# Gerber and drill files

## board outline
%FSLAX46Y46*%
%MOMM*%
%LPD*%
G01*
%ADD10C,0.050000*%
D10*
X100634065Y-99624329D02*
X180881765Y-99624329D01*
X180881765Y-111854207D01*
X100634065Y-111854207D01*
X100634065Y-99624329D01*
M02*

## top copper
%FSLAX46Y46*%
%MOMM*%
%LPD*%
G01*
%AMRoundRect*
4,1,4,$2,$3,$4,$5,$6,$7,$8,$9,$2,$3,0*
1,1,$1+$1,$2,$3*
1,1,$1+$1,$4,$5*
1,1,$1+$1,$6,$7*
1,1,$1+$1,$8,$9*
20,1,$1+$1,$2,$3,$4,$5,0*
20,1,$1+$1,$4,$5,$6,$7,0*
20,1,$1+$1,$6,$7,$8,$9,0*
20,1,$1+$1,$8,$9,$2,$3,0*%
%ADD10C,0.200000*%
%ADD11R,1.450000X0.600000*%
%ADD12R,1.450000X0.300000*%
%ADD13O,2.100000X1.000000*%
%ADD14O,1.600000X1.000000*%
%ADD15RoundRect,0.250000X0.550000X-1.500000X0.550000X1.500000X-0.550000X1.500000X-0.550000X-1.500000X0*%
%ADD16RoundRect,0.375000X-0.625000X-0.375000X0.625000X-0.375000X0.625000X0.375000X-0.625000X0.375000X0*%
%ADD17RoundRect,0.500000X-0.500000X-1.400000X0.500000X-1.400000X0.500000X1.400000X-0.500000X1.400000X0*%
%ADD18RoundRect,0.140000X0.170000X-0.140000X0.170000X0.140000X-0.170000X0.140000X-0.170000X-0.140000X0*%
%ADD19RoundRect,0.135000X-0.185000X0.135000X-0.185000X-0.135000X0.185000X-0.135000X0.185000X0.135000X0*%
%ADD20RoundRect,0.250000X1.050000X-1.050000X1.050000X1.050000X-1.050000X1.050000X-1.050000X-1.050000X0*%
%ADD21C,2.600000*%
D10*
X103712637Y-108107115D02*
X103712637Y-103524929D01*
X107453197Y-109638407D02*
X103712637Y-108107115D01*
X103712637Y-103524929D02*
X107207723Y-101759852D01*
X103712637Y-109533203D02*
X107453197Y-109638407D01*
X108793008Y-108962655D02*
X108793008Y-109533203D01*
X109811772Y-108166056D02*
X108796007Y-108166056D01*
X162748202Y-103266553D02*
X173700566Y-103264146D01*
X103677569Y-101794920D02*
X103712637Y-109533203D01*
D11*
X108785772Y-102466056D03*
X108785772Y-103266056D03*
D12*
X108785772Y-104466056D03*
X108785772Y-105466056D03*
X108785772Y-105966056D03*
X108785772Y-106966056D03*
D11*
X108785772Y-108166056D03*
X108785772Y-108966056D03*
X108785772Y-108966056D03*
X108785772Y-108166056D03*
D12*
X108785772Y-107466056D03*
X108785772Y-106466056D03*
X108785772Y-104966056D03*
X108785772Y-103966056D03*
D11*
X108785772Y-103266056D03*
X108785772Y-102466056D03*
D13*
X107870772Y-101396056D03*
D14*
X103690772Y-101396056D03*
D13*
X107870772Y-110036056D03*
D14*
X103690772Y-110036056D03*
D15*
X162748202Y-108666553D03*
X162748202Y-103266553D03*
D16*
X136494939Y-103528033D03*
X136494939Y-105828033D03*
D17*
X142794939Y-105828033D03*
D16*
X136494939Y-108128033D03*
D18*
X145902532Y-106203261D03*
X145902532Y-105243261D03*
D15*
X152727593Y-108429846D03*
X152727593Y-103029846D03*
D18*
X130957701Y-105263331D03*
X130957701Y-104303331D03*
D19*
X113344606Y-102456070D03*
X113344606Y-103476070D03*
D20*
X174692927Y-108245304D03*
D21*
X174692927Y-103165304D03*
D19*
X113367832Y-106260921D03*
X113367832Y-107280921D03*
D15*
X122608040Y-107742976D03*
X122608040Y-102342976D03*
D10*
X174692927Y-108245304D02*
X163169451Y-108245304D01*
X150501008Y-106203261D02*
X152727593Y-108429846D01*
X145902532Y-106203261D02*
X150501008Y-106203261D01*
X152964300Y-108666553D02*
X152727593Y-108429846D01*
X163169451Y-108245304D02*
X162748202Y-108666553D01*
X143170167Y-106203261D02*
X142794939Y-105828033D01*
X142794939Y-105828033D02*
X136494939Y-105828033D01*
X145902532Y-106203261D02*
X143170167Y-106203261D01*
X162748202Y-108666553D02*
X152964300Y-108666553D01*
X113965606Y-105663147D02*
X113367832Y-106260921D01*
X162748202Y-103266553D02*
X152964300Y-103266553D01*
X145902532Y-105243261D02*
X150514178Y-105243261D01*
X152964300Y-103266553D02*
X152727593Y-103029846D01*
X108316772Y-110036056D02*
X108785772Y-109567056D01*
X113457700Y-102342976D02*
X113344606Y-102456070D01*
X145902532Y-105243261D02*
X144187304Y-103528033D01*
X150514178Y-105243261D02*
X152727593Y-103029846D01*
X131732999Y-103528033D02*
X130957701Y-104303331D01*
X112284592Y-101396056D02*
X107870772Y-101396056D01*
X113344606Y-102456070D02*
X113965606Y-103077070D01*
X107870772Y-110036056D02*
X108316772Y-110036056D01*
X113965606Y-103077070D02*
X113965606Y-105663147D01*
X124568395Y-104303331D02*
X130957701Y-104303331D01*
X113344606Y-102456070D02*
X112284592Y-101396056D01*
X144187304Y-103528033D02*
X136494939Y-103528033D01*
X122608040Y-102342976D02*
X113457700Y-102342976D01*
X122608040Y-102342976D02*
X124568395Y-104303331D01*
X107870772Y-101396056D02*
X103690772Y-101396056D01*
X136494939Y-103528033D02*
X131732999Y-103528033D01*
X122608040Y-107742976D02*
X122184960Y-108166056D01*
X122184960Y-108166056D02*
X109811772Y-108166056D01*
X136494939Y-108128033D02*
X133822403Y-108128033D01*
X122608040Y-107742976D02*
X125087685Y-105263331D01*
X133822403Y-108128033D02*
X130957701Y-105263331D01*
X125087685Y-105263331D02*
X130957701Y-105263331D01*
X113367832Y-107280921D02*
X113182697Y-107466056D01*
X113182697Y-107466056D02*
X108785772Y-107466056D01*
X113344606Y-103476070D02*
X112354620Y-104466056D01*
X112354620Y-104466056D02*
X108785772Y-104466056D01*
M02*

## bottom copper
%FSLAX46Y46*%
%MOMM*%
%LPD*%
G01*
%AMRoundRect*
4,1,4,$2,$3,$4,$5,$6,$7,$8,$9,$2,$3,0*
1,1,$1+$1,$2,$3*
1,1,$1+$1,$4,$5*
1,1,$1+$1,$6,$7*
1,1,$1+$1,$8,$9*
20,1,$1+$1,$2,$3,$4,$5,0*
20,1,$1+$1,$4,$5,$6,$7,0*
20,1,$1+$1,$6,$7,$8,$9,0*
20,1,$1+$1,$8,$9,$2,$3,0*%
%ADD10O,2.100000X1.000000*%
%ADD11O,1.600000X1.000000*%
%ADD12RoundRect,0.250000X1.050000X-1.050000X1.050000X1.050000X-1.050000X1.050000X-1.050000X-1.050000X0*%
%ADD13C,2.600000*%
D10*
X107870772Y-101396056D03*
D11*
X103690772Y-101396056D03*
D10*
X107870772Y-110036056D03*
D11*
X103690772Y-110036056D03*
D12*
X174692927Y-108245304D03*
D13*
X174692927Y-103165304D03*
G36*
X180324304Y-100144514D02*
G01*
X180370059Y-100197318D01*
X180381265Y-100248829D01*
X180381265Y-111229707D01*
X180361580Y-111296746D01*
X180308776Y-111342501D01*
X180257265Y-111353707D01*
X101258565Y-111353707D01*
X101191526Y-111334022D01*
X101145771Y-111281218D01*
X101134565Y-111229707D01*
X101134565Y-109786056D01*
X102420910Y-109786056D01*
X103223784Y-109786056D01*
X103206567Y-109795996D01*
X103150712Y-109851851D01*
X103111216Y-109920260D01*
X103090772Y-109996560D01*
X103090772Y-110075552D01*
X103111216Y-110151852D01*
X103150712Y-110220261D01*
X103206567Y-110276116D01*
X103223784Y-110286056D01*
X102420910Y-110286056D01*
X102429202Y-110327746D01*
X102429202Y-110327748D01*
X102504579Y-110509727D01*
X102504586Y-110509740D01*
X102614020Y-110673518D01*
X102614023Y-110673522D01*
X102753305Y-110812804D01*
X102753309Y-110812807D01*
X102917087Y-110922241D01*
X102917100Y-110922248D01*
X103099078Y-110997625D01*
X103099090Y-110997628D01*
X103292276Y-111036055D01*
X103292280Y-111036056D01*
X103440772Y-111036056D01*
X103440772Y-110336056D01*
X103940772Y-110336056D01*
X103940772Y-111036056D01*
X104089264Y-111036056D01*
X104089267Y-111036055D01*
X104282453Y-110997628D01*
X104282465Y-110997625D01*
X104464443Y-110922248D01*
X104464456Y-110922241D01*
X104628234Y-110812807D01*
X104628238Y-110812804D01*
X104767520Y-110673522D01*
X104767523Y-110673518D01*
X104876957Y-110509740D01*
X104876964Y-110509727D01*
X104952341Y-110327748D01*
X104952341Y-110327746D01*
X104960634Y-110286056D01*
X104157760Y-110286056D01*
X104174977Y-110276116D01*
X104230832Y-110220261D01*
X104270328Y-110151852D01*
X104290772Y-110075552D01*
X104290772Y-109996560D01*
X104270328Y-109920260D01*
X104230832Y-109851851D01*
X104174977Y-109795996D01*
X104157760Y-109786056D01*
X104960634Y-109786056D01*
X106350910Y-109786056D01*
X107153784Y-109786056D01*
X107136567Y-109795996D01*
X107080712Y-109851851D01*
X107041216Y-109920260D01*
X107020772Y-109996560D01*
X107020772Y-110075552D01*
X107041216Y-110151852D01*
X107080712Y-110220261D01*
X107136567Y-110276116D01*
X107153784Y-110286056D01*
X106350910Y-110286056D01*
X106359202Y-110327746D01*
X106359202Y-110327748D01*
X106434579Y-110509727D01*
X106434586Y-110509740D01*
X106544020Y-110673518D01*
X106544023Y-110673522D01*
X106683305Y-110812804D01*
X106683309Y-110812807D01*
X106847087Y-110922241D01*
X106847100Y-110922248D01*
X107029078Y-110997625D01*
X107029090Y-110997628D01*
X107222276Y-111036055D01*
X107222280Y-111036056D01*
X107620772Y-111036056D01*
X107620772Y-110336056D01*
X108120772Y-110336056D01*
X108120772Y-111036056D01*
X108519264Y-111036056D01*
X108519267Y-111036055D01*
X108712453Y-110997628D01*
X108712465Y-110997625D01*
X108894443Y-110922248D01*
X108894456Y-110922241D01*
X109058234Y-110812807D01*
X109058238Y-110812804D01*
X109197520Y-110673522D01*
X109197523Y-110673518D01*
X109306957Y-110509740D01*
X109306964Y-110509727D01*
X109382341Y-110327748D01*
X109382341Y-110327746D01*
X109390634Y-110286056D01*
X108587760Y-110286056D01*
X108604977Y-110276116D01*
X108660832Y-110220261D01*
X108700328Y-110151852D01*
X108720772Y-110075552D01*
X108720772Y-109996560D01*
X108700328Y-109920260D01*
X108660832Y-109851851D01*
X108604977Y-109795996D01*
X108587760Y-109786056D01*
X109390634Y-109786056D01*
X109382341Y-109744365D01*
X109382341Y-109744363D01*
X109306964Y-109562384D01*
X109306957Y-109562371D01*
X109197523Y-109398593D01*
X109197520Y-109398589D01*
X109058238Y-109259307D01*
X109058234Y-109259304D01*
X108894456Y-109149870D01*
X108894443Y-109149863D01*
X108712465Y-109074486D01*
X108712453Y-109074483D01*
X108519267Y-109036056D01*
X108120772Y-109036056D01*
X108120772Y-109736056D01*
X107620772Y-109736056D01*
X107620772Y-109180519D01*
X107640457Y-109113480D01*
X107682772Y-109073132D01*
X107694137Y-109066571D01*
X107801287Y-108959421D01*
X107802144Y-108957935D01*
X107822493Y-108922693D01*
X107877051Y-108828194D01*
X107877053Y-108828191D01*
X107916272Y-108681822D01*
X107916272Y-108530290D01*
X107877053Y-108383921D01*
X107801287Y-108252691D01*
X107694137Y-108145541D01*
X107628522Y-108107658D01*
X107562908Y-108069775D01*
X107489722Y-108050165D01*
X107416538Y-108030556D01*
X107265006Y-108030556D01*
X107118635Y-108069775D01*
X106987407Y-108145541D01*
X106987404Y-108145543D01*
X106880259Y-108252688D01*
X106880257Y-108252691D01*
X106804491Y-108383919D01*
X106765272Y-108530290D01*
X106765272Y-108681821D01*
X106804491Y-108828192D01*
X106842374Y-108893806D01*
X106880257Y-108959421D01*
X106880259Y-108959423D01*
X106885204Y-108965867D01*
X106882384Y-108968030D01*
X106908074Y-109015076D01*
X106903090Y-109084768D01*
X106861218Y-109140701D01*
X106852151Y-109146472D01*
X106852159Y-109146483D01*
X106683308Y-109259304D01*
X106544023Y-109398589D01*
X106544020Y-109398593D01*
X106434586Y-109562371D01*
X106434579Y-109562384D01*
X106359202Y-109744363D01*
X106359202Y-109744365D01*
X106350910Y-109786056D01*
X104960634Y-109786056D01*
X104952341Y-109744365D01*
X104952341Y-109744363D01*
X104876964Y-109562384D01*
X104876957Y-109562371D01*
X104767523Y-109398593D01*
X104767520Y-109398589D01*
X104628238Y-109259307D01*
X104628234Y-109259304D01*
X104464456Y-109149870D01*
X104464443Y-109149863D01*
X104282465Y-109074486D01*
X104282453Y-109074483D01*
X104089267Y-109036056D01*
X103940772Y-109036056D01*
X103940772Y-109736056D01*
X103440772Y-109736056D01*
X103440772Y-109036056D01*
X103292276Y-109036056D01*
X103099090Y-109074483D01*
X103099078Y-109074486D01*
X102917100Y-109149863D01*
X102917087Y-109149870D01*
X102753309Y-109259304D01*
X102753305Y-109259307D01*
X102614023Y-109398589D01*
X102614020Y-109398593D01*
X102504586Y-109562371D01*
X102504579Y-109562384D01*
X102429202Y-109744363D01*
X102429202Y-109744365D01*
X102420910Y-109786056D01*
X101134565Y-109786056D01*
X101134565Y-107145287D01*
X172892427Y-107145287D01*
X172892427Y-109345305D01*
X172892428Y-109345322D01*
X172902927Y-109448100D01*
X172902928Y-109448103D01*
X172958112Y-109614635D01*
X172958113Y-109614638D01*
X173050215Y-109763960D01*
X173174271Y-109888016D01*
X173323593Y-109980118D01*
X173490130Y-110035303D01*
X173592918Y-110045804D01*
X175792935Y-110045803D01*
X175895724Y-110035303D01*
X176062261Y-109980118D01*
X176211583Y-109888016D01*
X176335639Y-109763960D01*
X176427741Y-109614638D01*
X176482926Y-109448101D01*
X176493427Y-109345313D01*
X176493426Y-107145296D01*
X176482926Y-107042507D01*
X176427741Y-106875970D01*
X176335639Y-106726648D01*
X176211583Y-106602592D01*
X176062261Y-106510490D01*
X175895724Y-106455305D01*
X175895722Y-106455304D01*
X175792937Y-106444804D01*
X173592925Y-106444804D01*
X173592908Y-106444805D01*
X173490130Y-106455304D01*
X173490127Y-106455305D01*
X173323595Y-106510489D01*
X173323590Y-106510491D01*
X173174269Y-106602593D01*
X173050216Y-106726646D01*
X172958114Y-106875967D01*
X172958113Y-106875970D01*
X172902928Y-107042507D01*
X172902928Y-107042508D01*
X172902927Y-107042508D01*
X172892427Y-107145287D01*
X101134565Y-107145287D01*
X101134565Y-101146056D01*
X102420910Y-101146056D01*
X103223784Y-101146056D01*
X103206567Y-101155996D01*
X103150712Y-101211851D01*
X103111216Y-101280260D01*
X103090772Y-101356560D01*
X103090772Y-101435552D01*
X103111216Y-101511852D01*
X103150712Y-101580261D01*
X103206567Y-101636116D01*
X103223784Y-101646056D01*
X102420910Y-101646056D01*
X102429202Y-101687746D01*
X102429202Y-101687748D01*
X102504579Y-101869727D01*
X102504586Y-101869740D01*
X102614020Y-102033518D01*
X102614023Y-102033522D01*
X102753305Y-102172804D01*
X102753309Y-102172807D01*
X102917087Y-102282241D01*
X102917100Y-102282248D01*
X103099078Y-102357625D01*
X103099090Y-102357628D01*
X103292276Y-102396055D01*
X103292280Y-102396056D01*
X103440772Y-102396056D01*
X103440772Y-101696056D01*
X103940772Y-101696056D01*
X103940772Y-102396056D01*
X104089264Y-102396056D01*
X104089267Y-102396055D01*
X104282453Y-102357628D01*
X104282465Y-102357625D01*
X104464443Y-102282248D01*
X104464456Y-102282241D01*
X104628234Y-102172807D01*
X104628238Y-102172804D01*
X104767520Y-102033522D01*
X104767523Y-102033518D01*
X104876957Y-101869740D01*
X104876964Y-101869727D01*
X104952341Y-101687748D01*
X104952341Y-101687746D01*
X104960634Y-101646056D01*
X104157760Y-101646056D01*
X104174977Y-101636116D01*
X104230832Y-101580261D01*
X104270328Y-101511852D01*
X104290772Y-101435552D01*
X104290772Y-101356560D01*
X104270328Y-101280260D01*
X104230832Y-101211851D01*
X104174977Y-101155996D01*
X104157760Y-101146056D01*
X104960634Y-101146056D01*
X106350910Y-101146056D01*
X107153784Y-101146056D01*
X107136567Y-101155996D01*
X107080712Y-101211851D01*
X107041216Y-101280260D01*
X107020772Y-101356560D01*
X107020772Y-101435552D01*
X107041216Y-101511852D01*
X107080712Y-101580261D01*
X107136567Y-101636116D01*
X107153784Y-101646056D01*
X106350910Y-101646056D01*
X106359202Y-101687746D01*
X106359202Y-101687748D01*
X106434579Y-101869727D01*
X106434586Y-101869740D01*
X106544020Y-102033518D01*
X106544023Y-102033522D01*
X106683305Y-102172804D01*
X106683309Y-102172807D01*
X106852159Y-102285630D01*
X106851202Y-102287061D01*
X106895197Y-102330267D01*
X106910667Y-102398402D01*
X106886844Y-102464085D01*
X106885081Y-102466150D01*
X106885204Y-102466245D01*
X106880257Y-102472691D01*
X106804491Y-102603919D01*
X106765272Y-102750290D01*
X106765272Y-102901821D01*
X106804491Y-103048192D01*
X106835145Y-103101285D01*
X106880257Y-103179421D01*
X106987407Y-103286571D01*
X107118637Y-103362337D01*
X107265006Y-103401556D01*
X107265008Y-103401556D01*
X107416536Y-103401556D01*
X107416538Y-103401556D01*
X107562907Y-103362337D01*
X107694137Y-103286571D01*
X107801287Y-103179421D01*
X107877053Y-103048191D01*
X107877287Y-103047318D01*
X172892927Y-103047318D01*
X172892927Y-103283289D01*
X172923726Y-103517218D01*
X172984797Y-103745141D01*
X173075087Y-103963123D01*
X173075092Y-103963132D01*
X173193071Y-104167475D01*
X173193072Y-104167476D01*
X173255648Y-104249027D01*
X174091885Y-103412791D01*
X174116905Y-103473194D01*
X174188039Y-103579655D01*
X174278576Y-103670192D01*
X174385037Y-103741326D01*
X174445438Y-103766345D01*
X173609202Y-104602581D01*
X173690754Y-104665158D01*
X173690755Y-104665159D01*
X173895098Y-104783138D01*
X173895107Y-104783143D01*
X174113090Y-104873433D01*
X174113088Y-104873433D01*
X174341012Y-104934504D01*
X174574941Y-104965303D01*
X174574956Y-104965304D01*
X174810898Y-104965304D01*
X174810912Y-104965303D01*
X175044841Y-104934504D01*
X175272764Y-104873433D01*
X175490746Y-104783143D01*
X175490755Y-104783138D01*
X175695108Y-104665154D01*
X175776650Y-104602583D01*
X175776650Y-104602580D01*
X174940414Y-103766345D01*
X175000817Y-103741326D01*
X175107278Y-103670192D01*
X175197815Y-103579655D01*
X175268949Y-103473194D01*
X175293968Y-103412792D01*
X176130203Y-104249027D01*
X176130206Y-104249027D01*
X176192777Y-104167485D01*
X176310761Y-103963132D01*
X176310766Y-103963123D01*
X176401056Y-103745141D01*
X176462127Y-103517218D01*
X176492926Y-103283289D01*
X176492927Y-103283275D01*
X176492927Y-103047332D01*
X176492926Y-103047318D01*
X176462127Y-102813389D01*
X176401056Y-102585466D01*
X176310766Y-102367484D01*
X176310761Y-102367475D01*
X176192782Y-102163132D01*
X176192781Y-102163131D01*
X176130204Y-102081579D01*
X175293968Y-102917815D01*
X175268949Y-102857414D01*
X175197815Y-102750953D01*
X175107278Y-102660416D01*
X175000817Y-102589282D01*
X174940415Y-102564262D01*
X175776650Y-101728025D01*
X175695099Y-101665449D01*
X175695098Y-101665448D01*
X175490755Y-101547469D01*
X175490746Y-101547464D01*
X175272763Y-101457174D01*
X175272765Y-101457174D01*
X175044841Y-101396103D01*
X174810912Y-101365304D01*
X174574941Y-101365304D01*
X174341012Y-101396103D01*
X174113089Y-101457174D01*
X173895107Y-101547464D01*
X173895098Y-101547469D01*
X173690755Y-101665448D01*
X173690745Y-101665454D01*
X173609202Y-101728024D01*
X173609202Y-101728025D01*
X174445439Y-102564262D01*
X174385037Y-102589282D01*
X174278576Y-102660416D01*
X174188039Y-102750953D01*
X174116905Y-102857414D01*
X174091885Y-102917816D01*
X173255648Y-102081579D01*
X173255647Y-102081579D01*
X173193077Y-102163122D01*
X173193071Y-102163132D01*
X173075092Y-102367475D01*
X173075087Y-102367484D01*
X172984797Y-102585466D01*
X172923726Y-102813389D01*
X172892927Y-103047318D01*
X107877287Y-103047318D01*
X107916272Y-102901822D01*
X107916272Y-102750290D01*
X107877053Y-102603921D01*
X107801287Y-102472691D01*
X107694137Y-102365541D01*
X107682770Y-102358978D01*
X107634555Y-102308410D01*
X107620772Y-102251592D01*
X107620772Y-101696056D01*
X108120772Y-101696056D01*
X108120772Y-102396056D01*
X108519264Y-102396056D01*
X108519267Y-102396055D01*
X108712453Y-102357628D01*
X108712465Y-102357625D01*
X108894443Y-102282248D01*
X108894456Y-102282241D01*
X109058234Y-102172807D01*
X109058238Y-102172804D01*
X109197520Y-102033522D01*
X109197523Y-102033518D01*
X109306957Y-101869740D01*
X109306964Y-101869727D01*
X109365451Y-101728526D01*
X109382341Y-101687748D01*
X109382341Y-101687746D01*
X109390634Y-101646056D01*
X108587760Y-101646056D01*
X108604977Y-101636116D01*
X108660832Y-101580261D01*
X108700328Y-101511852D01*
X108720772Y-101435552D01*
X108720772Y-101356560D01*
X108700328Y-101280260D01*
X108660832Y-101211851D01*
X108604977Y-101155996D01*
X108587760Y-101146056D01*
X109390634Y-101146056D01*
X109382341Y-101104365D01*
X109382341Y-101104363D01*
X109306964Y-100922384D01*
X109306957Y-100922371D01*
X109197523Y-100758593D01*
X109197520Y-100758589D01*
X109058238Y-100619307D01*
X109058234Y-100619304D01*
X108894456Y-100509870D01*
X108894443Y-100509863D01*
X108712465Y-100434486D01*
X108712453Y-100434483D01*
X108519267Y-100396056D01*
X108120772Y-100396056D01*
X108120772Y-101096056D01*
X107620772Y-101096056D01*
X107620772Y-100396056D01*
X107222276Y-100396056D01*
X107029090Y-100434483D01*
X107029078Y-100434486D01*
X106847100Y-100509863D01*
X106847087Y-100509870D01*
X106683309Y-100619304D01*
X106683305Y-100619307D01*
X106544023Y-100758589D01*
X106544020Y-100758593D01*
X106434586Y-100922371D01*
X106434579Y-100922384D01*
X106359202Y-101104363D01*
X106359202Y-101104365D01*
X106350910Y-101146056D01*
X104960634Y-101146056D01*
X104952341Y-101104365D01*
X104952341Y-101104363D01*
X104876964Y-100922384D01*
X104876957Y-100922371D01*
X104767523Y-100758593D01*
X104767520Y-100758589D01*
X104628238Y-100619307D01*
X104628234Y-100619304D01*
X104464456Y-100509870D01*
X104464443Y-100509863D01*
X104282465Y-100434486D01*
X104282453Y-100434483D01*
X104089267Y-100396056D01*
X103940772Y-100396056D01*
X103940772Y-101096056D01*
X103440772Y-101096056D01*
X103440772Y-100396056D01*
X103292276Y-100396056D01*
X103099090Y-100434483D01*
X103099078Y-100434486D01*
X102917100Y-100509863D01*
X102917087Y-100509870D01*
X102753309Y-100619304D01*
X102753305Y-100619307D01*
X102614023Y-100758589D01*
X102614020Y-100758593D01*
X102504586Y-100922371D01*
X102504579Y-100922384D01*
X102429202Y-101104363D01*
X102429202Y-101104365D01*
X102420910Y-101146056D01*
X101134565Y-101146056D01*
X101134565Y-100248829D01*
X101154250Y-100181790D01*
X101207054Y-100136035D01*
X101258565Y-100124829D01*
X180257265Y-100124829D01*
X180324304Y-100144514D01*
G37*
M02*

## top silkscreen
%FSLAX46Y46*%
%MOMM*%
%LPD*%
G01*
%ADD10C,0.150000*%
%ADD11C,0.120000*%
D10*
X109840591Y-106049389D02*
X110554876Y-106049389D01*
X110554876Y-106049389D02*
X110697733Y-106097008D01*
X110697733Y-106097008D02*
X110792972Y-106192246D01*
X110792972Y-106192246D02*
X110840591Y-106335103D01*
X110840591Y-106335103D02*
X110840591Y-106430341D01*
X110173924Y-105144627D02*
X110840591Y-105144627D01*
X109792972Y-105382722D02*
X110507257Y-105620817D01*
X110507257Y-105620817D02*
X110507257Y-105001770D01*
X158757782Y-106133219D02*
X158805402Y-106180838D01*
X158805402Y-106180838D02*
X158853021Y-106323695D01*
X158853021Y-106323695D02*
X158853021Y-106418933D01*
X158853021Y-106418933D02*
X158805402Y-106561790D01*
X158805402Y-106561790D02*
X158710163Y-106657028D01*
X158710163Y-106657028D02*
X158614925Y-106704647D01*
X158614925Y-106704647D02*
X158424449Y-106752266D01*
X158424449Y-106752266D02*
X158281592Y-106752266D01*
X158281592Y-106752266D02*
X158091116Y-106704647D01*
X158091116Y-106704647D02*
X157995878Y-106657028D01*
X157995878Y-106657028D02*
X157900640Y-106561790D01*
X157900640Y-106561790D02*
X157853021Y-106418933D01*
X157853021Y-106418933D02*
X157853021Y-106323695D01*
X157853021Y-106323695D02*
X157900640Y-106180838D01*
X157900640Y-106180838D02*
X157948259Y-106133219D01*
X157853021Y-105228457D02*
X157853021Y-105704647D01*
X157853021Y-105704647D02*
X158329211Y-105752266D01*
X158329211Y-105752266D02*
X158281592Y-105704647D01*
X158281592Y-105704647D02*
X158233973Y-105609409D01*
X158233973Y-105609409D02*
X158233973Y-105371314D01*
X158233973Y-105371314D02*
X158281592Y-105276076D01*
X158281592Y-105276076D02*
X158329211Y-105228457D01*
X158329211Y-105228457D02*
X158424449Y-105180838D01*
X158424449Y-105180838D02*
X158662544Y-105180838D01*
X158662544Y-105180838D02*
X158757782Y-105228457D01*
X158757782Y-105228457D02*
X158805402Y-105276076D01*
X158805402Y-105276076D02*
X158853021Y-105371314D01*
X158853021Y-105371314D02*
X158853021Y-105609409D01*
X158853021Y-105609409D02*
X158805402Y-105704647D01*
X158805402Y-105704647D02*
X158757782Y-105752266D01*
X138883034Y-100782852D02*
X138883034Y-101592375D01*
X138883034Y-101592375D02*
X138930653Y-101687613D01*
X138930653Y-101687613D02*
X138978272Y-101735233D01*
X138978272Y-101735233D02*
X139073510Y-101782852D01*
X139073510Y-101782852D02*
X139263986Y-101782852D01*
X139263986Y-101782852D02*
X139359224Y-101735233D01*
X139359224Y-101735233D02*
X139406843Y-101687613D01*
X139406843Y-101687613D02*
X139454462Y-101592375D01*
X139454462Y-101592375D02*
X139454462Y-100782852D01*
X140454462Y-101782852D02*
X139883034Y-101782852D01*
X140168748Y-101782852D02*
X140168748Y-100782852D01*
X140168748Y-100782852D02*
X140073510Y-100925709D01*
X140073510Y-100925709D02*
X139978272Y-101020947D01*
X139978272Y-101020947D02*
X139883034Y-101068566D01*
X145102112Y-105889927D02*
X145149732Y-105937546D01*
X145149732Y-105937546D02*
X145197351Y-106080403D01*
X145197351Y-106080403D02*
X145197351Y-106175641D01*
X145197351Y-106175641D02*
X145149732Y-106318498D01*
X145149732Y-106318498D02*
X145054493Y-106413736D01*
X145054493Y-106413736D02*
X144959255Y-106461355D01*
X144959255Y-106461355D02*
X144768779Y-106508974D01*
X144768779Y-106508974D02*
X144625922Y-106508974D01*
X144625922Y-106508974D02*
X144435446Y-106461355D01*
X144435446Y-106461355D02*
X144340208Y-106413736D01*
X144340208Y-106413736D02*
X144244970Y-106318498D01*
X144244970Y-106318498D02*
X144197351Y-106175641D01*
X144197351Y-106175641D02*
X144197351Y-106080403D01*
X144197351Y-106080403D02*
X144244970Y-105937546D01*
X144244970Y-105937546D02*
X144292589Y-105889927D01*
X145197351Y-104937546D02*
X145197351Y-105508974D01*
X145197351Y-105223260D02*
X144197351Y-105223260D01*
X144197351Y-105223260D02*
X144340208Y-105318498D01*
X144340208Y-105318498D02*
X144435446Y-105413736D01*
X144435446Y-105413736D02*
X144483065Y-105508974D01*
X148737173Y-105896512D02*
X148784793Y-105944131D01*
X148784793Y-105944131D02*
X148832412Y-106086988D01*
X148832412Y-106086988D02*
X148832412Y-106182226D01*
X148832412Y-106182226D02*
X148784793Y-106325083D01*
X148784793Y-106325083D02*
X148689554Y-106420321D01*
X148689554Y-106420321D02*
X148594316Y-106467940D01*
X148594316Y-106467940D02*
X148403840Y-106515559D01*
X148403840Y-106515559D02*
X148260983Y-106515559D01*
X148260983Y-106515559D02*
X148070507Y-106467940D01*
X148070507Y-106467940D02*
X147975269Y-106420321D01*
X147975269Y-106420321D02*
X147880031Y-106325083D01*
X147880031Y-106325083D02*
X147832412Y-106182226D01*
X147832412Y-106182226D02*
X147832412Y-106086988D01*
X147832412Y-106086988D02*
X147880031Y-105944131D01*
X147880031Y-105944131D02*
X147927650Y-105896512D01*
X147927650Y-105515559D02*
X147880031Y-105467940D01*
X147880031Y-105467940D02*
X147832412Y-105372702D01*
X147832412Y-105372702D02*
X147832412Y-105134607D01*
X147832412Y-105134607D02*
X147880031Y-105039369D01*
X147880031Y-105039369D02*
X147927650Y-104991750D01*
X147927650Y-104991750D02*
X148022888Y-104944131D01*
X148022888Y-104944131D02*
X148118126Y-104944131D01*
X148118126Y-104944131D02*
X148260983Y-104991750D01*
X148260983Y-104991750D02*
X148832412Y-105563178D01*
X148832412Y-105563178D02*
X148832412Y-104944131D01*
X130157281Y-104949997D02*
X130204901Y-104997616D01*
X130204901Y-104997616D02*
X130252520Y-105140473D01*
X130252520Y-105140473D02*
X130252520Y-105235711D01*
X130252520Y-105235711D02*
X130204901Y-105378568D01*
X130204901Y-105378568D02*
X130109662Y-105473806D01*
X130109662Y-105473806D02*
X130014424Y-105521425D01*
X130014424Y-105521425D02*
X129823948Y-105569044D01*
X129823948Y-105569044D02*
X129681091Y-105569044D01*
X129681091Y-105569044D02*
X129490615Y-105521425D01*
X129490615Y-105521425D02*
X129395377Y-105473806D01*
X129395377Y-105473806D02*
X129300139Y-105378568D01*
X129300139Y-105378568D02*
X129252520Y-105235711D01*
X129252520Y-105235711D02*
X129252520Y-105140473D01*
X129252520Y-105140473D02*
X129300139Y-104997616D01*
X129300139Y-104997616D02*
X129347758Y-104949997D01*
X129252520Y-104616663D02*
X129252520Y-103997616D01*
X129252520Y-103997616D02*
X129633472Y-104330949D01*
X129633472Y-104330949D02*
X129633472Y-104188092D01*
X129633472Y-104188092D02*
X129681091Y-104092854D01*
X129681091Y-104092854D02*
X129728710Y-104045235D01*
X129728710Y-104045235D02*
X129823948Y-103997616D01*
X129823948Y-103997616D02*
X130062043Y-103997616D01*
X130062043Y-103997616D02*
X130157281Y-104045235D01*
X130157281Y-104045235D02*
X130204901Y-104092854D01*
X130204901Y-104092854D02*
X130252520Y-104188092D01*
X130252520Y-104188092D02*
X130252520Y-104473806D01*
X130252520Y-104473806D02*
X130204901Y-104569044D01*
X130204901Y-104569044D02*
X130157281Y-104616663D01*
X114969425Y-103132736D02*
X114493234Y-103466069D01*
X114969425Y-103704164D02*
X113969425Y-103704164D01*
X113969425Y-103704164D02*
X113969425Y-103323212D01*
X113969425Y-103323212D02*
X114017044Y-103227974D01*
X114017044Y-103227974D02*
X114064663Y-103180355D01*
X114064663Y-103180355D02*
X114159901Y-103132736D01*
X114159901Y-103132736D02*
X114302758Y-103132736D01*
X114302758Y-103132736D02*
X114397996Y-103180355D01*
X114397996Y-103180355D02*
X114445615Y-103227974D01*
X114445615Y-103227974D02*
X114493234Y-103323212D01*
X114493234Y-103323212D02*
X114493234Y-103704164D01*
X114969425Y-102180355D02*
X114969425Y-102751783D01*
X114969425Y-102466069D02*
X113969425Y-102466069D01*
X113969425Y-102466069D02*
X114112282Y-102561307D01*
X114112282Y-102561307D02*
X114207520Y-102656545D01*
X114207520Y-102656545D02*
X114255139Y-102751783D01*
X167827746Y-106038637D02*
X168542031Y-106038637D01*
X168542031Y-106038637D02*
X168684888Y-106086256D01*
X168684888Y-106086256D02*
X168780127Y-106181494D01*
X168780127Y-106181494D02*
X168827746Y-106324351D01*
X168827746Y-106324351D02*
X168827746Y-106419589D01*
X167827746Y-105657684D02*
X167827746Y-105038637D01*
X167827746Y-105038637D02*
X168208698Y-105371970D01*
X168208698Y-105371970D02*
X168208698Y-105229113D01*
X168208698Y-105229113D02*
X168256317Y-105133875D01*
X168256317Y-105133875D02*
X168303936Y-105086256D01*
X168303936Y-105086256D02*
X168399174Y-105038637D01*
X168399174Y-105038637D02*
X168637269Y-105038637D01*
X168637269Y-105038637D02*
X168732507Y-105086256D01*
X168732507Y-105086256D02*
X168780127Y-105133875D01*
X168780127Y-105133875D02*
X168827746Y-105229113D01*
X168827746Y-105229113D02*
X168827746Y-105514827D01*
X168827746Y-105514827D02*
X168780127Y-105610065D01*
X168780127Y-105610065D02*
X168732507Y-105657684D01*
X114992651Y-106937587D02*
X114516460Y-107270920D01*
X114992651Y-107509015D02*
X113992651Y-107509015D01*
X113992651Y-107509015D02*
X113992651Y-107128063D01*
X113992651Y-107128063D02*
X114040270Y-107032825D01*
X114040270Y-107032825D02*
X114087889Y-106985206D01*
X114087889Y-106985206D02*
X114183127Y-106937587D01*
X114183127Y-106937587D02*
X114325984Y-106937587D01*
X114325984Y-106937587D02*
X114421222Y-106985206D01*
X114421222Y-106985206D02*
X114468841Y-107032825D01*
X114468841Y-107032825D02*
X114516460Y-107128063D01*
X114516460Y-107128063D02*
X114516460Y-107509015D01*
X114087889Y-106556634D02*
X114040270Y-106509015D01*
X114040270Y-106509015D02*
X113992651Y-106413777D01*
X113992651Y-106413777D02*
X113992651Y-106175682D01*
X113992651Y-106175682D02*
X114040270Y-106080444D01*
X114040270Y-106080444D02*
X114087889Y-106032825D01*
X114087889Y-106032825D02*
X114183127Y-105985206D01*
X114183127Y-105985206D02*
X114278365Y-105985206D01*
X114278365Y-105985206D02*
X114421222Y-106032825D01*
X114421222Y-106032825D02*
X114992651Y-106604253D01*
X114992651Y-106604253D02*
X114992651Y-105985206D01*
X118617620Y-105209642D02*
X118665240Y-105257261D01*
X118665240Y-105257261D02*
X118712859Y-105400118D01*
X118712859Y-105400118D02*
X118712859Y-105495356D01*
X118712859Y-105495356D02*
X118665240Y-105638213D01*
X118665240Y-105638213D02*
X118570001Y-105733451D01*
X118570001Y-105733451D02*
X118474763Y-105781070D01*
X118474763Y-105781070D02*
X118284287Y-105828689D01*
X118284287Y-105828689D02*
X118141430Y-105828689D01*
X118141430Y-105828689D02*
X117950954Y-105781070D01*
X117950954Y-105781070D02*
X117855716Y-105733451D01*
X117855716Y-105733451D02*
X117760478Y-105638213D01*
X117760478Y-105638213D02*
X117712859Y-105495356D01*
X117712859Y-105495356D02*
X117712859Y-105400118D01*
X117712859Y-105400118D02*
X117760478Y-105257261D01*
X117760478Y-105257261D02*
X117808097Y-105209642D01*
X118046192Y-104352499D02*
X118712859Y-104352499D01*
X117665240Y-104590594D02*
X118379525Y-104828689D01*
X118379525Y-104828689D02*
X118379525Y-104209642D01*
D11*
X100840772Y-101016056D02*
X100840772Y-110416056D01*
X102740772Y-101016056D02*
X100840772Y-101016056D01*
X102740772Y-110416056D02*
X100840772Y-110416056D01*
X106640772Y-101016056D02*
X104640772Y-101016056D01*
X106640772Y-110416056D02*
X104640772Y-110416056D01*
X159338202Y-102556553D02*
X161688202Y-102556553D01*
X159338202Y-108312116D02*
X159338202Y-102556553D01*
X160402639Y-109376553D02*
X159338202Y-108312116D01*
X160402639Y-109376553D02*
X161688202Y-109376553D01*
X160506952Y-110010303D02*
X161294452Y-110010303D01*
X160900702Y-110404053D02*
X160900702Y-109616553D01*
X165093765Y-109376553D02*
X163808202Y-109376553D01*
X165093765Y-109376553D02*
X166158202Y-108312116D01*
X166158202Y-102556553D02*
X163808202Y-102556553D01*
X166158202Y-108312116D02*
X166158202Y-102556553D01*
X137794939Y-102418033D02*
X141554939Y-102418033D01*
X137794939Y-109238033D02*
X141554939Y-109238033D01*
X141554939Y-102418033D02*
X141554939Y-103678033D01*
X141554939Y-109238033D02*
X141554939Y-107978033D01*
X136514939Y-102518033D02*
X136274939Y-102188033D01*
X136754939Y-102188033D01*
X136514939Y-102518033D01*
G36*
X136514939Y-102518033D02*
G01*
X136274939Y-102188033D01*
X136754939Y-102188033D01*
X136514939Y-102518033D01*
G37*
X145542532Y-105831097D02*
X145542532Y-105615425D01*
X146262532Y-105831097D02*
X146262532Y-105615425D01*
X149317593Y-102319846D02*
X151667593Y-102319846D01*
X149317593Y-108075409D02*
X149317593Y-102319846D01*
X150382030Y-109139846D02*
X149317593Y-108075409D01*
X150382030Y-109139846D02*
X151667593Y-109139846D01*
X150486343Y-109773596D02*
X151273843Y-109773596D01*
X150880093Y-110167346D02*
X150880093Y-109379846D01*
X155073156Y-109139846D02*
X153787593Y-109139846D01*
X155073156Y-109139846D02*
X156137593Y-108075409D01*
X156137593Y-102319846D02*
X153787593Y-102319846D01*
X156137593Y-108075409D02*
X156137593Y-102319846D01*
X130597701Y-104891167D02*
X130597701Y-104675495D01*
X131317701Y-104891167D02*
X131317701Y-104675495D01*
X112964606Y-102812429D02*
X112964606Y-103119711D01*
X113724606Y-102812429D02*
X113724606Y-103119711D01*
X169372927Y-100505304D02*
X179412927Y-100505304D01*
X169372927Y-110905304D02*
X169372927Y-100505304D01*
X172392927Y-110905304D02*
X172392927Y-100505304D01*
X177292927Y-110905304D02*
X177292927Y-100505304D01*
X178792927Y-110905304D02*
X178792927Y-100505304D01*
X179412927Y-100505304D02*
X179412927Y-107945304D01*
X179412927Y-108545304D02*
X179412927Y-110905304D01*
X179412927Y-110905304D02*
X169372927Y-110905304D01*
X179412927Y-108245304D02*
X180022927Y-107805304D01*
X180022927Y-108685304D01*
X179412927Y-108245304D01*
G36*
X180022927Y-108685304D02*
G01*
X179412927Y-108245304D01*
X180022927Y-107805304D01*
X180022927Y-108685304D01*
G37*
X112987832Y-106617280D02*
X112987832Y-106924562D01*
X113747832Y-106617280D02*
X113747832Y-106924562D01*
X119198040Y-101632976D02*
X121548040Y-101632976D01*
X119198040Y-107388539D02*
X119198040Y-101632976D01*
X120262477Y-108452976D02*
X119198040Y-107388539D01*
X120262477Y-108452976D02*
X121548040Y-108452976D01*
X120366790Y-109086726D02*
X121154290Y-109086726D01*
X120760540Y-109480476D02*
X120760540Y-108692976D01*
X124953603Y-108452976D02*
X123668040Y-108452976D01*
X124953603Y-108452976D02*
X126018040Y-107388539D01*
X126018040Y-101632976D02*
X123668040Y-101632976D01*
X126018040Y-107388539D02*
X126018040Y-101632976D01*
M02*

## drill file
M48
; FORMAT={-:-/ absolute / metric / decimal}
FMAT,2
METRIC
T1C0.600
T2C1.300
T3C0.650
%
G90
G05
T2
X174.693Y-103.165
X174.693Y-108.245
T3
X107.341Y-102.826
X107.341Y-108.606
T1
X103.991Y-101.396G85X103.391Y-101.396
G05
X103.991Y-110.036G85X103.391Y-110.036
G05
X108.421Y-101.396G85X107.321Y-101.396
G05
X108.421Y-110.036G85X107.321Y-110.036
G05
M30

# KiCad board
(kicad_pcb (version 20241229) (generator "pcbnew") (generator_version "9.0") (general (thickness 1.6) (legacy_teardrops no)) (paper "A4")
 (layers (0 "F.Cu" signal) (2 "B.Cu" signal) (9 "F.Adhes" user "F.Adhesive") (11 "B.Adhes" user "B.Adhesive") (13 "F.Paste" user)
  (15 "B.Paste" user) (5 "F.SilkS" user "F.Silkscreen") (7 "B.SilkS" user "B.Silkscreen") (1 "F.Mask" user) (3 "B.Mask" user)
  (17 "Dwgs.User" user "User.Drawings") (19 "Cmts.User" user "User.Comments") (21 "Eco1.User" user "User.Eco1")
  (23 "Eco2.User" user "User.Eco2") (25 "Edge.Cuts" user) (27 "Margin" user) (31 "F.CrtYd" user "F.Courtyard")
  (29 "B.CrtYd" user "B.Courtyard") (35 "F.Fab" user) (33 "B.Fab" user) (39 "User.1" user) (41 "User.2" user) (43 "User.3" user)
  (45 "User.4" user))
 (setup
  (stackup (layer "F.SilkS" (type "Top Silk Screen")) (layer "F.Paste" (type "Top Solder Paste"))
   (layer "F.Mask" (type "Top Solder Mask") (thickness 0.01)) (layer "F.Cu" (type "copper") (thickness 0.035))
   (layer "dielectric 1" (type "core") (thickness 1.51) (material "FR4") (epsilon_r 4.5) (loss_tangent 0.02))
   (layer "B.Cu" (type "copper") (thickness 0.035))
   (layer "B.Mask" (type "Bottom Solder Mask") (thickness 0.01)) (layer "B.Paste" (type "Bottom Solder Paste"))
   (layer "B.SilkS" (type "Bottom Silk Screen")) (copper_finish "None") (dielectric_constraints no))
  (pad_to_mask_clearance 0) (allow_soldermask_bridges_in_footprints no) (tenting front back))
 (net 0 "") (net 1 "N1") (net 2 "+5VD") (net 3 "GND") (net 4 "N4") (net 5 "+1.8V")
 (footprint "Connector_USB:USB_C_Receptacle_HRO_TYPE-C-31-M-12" (layer "F.Cu") (at 104.740772 105.716056 -90)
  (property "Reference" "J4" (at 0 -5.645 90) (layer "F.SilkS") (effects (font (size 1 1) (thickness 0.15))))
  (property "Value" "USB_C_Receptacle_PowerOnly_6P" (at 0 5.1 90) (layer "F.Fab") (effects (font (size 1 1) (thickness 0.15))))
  (fp_line (start -4.7 3.9) (end 4.7 3.9) (stroke (width 0.12) (type solid)) (layer "F.SilkS"))
  (fp_line (start -4.7 2) (end -4.7 3.9) (stroke (width 0.12) (type solid)) (layer "F.SilkS"))
  (fp_line (start 4.7 2) (end 4.7 3.9) (stroke (width 0.12) (type solid)) (layer "F.SilkS"))
  (fp_line (start -4.7 -1.9) (end -4.7 0.1) (stroke (width 0.12) (type solid)) (layer "F.SilkS"))
  (fp_line (start 4.7 -1.9) (end 4.7 0.1) (stroke (width 0.12) (type solid)) (layer "F.SilkS"))
  (pad "" np_thru_hole circle (at -2.89 -2.6 270) (size 0.65 0.65) (drill 0.65) (layers "*.Cu" "*.Mask"))
  (pad "" np_thru_hole circle (at 2.89 -2.6 270) (size 0.65 0.65) (drill 0.65) (layers "*.Cu" "*.Mask"))
  (pad "A1" smd rect (at -3.25 -4.045 270) (size 0.6 1.45) (layers "F.Cu" "F.Mask" "F.Paste"))
  (pad "A4" smd rect (at -2.45 -4.045 270) (size 0.6 1.45) (layers "F.Cu" "F.Mask" "F.Paste"))
  (pad "A5" smd rect (at -1.25 -4.045 270) (size 0.3 1.45) (layers "F.Cu" "F.Mask" "F.Paste") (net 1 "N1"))
  (pad "A6" smd rect (at -0.25 -4.045 270) (size 0.3 1.45) (layers "F.Cu" "F.Mask" "F.Paste"))
  (pad "A7" smd rect (at 0.25 -4.045 270) (size 0.3 1.45) (layers "F.Cu" "F.Mask" "F.Paste"))
  (pad "A8" smd rect (at 1.25 -4.045 270) (size 0.3 1.45) (layers "F.Cu" "F.Mask" "F.Paste"))
  (pad "A9" smd rect (at 2.45 -4.045 270) (size 0.6 1.45) (layers "F.Cu" "F.Mask" "F.Paste") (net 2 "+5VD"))
  (pad "A12" smd rect (at 3.25 -4.045 270) (size 0.6 1.45) (layers "F.Cu" "F.Mask" "F.Paste") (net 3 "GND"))
  (pad "B1" smd rect (at 3.25 -4.045 270) (size 0.6 1.45) (layers "F.Cu" "F.Mask" "F.Paste"))
  (pad "B4" smd rect (at 2.45 -4.045 270) (size 0.6 1.45) (layers "F.Cu" "F.Mask" "F.Paste"))
  (pad "B5" smd rect (at 1.75 -4.045 270) (size 0.3 1.45) (layers "F.Cu" "F.Mask" "F.Paste") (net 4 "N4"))
  (pad "B6" smd rect (at 0.75 -4.045 270) (size 0.3 1.45) (layers "F.Cu" "F.Mask" "F.Paste"))
  (pad "B7" smd rect (at -0.75 -4.045 270) (size 0.3 1.45) (layers "F.Cu" "F.Mask" "F.Paste"))
  (pad "B8" smd rect (at -1.75 -4.045 270) (size 0.3 1.45) (layers "F.Cu" "F.Mask" "F.Paste"))
  (pad "B9" smd rect (at -2.45 -4.045 270) (size 0.6 1.45) (layers "F.Cu" "F.Mask" "F.Paste") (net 2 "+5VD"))
  (pad "B12" smd rect (at -3.25 -4.045 270) (size 0.6 1.45) (layers "F.Cu" "F.Mask" "F.Paste") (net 3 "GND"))
  (pad "S1" thru_hole oval (at -4.32 -3.13 270) (size 1 2.1) (drill oval 0.6 1.7) (layers "*.Cu" "*.Mask") (remove_unused_layers no)
   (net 3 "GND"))
  (pad "S1" thru_hole oval (at -4.32 1.05 270) (size 1 1.6) (drill oval 0.6 1.2) (layers "*.Cu" "*.Mask") (remove_unused_layers no)
   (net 3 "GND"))
  (pad "S1" thru_hole oval (at 4.32 -3.13 270) (size 1 2.1) (drill oval 0.6 1.7) (layers "*.Cu" "*.Mask") (remove_unused_layers no)
   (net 3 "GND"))
  (pad "S1" thru_hole oval (at 4.32 1.05 270) (size 1 1.6) (drill oval 0.6 1.2) (layers "*.Cu" "*.Mask") (remove_unused_layers no)
   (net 3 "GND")))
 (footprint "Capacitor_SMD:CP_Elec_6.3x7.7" (layer "F.Cu") (at 162.748202 105.966553 90)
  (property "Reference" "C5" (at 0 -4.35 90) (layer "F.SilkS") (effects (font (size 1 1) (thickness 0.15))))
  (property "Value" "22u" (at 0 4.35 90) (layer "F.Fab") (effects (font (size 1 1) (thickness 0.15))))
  (fp_line (start 3.41 -3.41) (end 3.41 -1.06) (stroke (width 0.12) (type solid)) (layer "F.SilkS"))
  (fp_line (start -2.345563 -3.41) (end 3.41 -3.41) (stroke (width 0.12) (type solid)) (layer "F.SilkS"))
  (fp_line (start -3.41 -2.345563) (end -2.345563 -3.41) (stroke (width 0.12) (type solid)) (layer "F.SilkS"))
  (fp_line (start -3.41 -2.345563) (end -3.41 -1.06) (stroke (width 0.12) (type solid)) (layer "F.SilkS"))
  (fp_line (start -4.04375 -2.24125) (end -4.04375 -1.45375) (stroke (width 0.12) (type solid)) (layer "F.SilkS"))
  (fp_line (start -4.4375 -1.8475) (end -3.65 -1.8475) (stroke (width 0.12) (type solid)) (layer "F.SilkS"))
  (fp_line (start -3.41 2.345563) (end -3.41 1.06) (stroke (width 0.12) (type solid)) (layer "F.SilkS"))
  (fp_line (start -3.41 2.345563) (end -2.345563 3.41) (stroke (width 0.12) (type solid)) (layer "F.SilkS"))
  (fp_line (start 3.41 3.41) (end 3.41 1.06) (stroke (width 0.12) (type solid)) (layer "F.SilkS"))
  (fp_line (start -2.345563 3.41) (end 3.41 3.41) (stroke (width 0.12) (type solid)) (layer "F.SilkS"))
  (pad "1" smd roundrect (at -2.7 0 90) (size 3.5 1.6) (layers "F.Cu" "F.Mask" "F.Paste") (roundrect_rratio 0.15625) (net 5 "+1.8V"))
  (pad "2" smd roundrect (at 2.7 0 90) (size 3.5 1.6) (layers "F.Cu" "F.Mask" "F.Paste") (roundrect_rratio 0.15625) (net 3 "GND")))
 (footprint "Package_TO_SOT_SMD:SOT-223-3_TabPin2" (layer "F.Cu") (at 139.644939 105.828033)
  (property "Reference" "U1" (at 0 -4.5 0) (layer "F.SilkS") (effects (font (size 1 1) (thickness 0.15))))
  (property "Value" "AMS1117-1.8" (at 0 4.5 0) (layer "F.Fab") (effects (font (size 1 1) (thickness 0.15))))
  (fp_line (start -1.85 -3.41) (end 1.91 -3.41) (stroke (width 0.12) (type solid)) (layer "F.SilkS"))
  (fp_line (start -1.85 3.41) (end 1.91 3.41) (stroke (width 0.12) (type solid)) (layer "F.SilkS"))
  (fp_line (start 1.91 -3.41) (end 1.91 -2.15) (stroke (width 0.12) (type solid)) (layer "F.SilkS"))
  (fp_line (start 1.91 3.41) (end 1.91 2.15) (stroke (width 0.12) (type solid)) (layer "F.SilkS"))
  (fp_poly
   (pts (xy -3.13 -3.31) (xy -3.37 -3.64) (xy -2.89 -3.64) (xy -3.13 -3.31)) (stroke (width 0.12) (type solid)) (fill yes) (layer "F.SilkS"))
  (pad "1" smd roundrect (at -3.15 -2.3) (size 2 1.5) (layers "F.Cu" "F.Mask" "F.Paste") (roundrect_rratio 0.25) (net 3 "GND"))
  (pad "2" smd roundrect (at -3.15 0) (size 2 1.5) (layers "F.Cu" "F.Mask" "F.Paste") (roundrect_rratio 0.25) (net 5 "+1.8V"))
  (pad "2" smd roundrect (at 3.15 0) (size 2 3.8) (layers "F.Cu" "F.Mask" "F.Paste") (roundrect_rratio 0.25) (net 5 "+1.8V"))
  (pad "3" smd roundrect (at -3.15 2.3) (size 2 1.5) (layers "F.Cu" "F.Mask" "F.Paste") (roundrect_rratio 0.25) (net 2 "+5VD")))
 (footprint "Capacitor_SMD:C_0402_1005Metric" (layer "F.Cu") (at 145.902532 105.723261 90)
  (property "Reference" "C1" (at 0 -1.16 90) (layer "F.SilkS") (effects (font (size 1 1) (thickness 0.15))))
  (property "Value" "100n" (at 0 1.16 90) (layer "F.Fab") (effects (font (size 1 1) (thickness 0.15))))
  (fp_line (start -0.107836 -0.36) (end 0.107836 -0.36) (stroke (width 0.12) (type solid)) (layer "F.SilkS"))
  (fp_line (start -0.107836 0.36) (end 0.107836 0.36) (stroke (width 0.12) (type solid)) (layer "F.SilkS"))
  (pad "1" smd roundrect (at -0.48 0 90) (size 0.56 0.62) (layers "F.Cu" "F.Mask" "F.Paste") (roundrect_rratio 0.25) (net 5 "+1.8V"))
  (pad "2" smd roundrect (at 0.48 0 90) (size 0.56 0.62) (layers "F.Cu" "F.Mask" "F.Paste") (roundrect_rratio 0.25) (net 3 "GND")))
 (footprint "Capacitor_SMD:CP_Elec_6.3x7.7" (layer "F.Cu") (at 152.727593 105.729846 90)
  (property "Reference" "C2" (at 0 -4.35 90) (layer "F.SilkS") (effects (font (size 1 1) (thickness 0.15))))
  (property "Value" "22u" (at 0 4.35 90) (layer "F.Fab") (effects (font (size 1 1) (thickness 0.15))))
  (fp_line (start 3.41 -3.41) (end 3.41 -1.06) (stroke (width 0.12) (type solid)) (layer "F.SilkS"))
  (fp_line (start -2.345563 -3.41) (end 3.41 -3.41) (stroke (width 0.12) (type solid)) (layer "F.SilkS"))
  (fp_line (start -3.41 -2.345563) (end -2.345563 -3.41) (stroke (width 0.12) (type solid)) (layer "F.SilkS"))
  (fp_line (start -3.41 -2.345563) (end -3.41 -1.06) (stroke (width 0.12) (type solid)) (layer "F.SilkS"))
  (fp_line (start -4.04375 -2.24125) (end -4.04375 -1.45375) (stroke (width 0.12) (type solid)) (layer "F.SilkS"))
  (fp_line (start -4.4375 -1.8475) (end -3.65 -1.8475) (stroke (width 0.12) (type solid)) (layer "F.SilkS"))
  (fp_line (start -3.41 2.345563) (end -3.41 1.06) (stroke (width 0.12) (type solid)) (layer "F.SilkS"))
  (fp_line (start -3.41 2.345563) (end -2.345563 3.41) (stroke (width 0.12) (type solid)) (layer "F.SilkS"))
  (fp_line (start 3.41 3.41) (end 3.41 1.06) (stroke (width 0.12) (type solid)) (layer "F.SilkS"))
  (fp_line (start -2.345563 3.41) (end 3.41 3.41) (stroke (width 0.12) (type solid)) (layer "F.SilkS"))
  (pad "1" smd roundrect (at -2.7 0 90) (size 3.5 1.6) (layers "F.Cu" "F.Mask" "F.Paste") (roundrect_rratio 0.15625) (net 5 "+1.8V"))
  (pad "2" smd roundrect (at 2.7 0 90) (size 3.5 1.6) (layers "F.Cu" "F.Mask" "F.Paste") (roundrect_rratio 0.15625) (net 3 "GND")))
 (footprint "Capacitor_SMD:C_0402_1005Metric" (layer "F.Cu") (at 130.957701 104.783331 90)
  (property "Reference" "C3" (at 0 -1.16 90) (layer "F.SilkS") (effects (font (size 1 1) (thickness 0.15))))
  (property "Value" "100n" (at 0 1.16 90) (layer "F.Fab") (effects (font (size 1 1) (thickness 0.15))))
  (fp_line (start -0.107836 -0.36) (end 0.107836 -0.36) (stroke (width 0.12) (type solid)) (layer "F.SilkS"))
  (fp_line (start -0.107836 0.36) (end 0.107836 0.36) (stroke (width 0.12) (type solid)) (layer "F.SilkS"))
  (pad "1" smd roundrect (at -0.48 0 90) (size 0.56 0.62) (layers "F.Cu" "F.Mask" "F.Paste") (roundrect_rratio 0.25) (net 2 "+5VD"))
  (pad "2" smd roundrect (at 0.48 0 90) (size 0.56 0.62) (layers "F.Cu" "F.Mask" "F.Paste") (roundrect_rratio 0.25) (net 3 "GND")))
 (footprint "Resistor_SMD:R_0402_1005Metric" (layer "F.Cu") (at 113.344606 102.96607 -90)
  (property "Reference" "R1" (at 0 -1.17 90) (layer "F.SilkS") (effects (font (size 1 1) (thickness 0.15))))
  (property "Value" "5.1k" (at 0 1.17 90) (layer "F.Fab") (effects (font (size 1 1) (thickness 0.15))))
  (fp_line (start -0.153641 0.38) (end 0.153641 0.38) (stroke (width 0.12) (type solid)) (layer "F.SilkS"))
  (fp_line (start -0.153641 -0.38) (end 0.153641 -0.38) (stroke (width 0.12) (type solid)) (layer "F.SilkS"))
  (pad "1" smd roundrect (at -0.51 0 270) (size 0.54 0.64) (layers "F.Cu" "F.Mask" "F.Paste") (roundrect_rratio 0.25) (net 3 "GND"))
  (pad "2" smd roundrect (at 0.51 0 270) (size 0.54 0.64) (layers "F.Cu" "F.Mask" "F.Paste") (roundrect_rratio 0.25) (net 1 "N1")))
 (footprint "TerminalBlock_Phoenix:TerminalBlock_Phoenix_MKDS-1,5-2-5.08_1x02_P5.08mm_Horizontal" (layer "F.Cu")
  (at 174.692927 108.245304 90)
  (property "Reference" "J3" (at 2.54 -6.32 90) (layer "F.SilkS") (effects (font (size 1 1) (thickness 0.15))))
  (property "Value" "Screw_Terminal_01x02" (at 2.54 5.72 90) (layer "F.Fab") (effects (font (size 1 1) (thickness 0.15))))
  (fp_line (start 7.74 -5.32) (end 7.74 4.72) (stroke (width 0.12) (type solid)) (layer "F.SilkS"))
  (fp_line (start -2.66 -5.32) (end 7.74 -5.32) (stroke (width 0.12) (type solid)) (layer "F.SilkS"))
  (fp_line (start -2.66 -2.3) (end 7.74 -2.3) (stroke (width 0.12) (type solid)) (layer "F.SilkS"))
  (fp_line (start -2.66 2.6) (end 7.74 2.6) (stroke (width 0.12) (type solid)) (layer "F.SilkS"))
  (fp_line (start -2.66 4.1) (end 7.74 4.1) (stroke (width 0.12) (type solid)) (layer "F.SilkS"))
  (fp_line (start 7.74 4.72) (end 0.3 4.72) (stroke (width 0.12) (type solid)) (layer "F.SilkS"))
  (fp_line (start -0.3 4.72) (end -2.66 4.72) (stroke (width 0.12) (type solid)) (layer "F.SilkS"))
  (fp_line (start -2.66 4.72) (end -2.66 -5.32) (stroke (width 0.12) (type solid)) (layer "F.SilkS"))
  (fp_poly (pts (xy 0 4.72) (xy 0.44 5.33) (xy -0.44 5.33)) (stroke (width 0.12) (type solid)) (fill yes) (layer "F.SilkS"))
  (pad "1" thru_hole roundrect (at 0 0 90) (size 2.6 2.6) (drill 1.3) (layers "*.Cu" "*.Mask") (remove_unused_layers no)
   (roundrect_rratio 0.096154) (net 5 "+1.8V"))
  (pad "2" thru_hole circle (at 5.08 0 90) (size 2.6 2.6) (drill 1.3) (layers "*.Cu" "*.Mask") (remove_unused_layers no) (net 3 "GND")))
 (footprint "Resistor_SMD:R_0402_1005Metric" (layer "F.Cu") (at 113.367832 106.770921 -90)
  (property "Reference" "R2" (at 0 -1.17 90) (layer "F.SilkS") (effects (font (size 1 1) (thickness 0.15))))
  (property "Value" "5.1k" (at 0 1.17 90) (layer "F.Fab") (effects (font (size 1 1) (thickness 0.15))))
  (fp_line (start -0.153641 0.38) (end 0.153641 0.38) (stroke (width 0.12) (type solid)) (layer "F.SilkS"))
  (fp_line (start -0.153641 -0.38) (end 0.153641 -0.38) (stroke (width 0.12) (type solid)) (layer "F.SilkS"))
  (pad "1" smd roundrect (at -0.51 0 270) (size 0.54 0.64) (layers "F.Cu" "F.Mask" "F.Paste") (roundrect_rratio 0.25) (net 3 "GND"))
  (pad "2" smd roundrect (at 0.51 0 270) (size 0.54 0.64) (layers "F.Cu" "F.Mask" "F.Paste") (roundrect_rratio 0.25) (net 4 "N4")))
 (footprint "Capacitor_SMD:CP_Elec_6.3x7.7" (layer "F.Cu") (at 122.60804 105.042976 90)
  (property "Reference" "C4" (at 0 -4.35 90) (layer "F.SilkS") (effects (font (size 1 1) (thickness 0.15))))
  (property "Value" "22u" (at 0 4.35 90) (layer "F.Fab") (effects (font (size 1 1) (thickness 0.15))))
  (fp_line (start 3.41 -3.41) (end 3.41 -1.06) (stroke (width 0.12) (type solid)) (layer "F.SilkS"))
  (fp_line (start -2.345563 -3.41) (end 3.41 -3.41) (stroke (width 0.12) (type solid)) (layer "F.SilkS"))
  (fp_line (start -3.41 -2.345563) (end -2.345563 -3.41) (stroke (width 0.12) (type solid)) (layer "F.SilkS"))
  (fp_line (start -3.41 -2.345563) (end -3.41 -1.06) (stroke (width 0.12) (type solid)) (layer "F.SilkS"))
  (fp_line (start -4.04375 -2.24125) (end -4.04375 -1.45375) (stroke (width 0.12) (type solid)) (layer "F.SilkS"))
  (fp_line (start -4.4375 -1.8475) (end -3.65 -1.8475) (stroke (width 0.12) (type solid)) (layer "F.SilkS"))
  (fp_line (start -3.41 2.345563) (end -3.41 1.06) (stroke (width 0.12) (type solid)) (layer "F.SilkS"))
  (fp_line (start -3.41 2.345563) (end -2.345563 3.41) (stroke (width 0.12) (type solid)) (layer "F.SilkS"))
  (fp_line (start 3.41 3.41) (end 3.41 1.06) (stroke (width 0.12) (type solid)) (layer "F.SilkS"))
  (fp_line (start -2.345563 3.41) (end 3.41 3.41) (stroke (width 0.12) (type solid)) (layer "F.SilkS"))
  (pad "1" smd roundrect (at -2.7 0 90) (size 3.5 1.6) (layers "F.Cu" "F.Mask" "F.Paste") (roundrect_rratio 0.15625) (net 2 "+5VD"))
  (pad "2" smd roundrect (at 2.7 0 90) (size 3.5 1.6) (layers "F.Cu" "F.Mask" "F.Paste") (roundrect_rratio 0.15625) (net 3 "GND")))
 (gr_line (start 103.712637 108.107115) (end 103.712637 103.524929) (stroke (width 0.2) (type default)) (layer "F.Cu") (net 3))
 (gr_line (start 107.453197 109.638407) (end 103.712637 108.107115) (stroke (width 0.2) (type default)) (layer "F.Cu") (net 3))
 (gr_line (start 103.712637 103.524929) (end 107.207723 101.759852) (stroke (width 0.2) (type default)) (layer "F.Cu") (net 3))
 (gr_line (start 103.712637 109.533203) (end 107.453197 109.638407) (stroke (width 0.2) (type default)) (layer "F.Cu") (net 3))
 (gr_line (start 108.793008 108.962655) (end 108.793008 109.533203) (stroke (width 0.2) (type default)) (layer "F.Cu") (net 3))
 (gr_line (start 109.811772 108.166056) (end 108.796007 108.166056) (stroke (width 0.2) (type default)) (layer "F.Cu") (net 2))
 (gr_line (start 162.748202 103.266553) (end 173.700566 103.264146) (stroke (width 0.2) (type default)) (layer "F.Cu") (net 3))
 (gr_line (start 103.677569 101.79492) (end 103.712637 109.533203) (stroke (width 0.2) (type default)) (layer "F.Cu") (net 3))
 (gr_rect (start 100.634065 99.624329) (end 180.881765 111.854207) (stroke (width 0.05) (type default)) (fill no) (layer "Edge.Cuts"))
 (segment (start 174.692927 108.245304) (end 163.169451 108.245304) (width 0.2) (layer "F.Cu") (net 5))
 (segment (start 150.501008 106.203261) (end 152.727593 108.429846) (width 0.2) (layer "F.Cu") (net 5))
 (segment (start 145.902532 106.203261) (end 150.501008 106.203261) (width 0.2) (layer "F.Cu") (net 5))
 (segment (start 152.9643 108.666553) (end 152.727593 108.429846) (width 0.2) (layer "F.Cu") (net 5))
 (segment (start 163.169451 108.245304) (end 162.748202 108.666553) (width 0.2) (layer "F.Cu") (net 5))
 (segment (start 143.170167 106.203261) (end 142.794939 105.828033) (width 0.2) (layer "F.Cu") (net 5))
 (segment (start 142.794939 105.828033) (end 136.494939 105.828033) (width 0.2) (layer "F.Cu") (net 5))
 (segment (start 145.902532 106.203261) (end 143.170167 106.203261) (width 0.2) (layer "F.Cu") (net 5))
 (segment (start 162.748202 108.666553) (end 152.9643 108.666553) (width 0.2) (layer "F.Cu") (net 5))
 (segment (start 113.965606 105.663147) (end 113.367832 106.260921) (width 0.2) (layer "F.Cu") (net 3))
 (segment (start 162.748202 103.266553) (end 152.9643 103.266553) (width 0.2) (layer "F.Cu") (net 3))
 (segment (start 145.902532 105.243261) (end 150.514178 105.243261) (width 0.2) (layer "F.Cu") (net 3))
 (segment (start 152.9643 103.266553) (end 152.727593 103.029846) (width 0.2) (layer "F.Cu") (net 3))
 (segment (start 108.316772 110.036056) (end 108.785772 109.567056) (width 0.2) (layer "F.Cu") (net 3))
 (segment (start 113.4577 102.342976) (end 113.344606 102.45607) (width 0.2) (layer "F.Cu") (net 3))
 (segment (start 145.902532 105.243261) (end 144.187304 103.528033) (width 0.2) (layer "F.Cu") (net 3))
 (segment (start 150.514178 105.243261) (end 152.727593 103.029846) (width 0.2) (layer "F.Cu") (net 3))
 (segment (start 131.732999 103.528033) (end 130.957701 104.303331) (width 0.2) (layer "F.Cu") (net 3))
 (segment (start 112.284592 101.396056) (end 107.870772 101.396056) (width 0.2) (layer "F.Cu") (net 3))
 (segment (start 113.344606 102.45607) (end 113.965606 103.07707) (width 0.2) (layer "F.Cu") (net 3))
 (segment (start 107.870772 110.036056) (end 108.316772 110.036056) (width 0.2) (layer "F.Cu") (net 3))
 (segment (start 113.965606 103.07707) (end 113.965606 105.663147) (width 0.2) (layer "F.Cu") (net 3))
 (segment (start 124.568395 104.303331) (end 130.957701 104.303331) (width 0.2) (layer "F.Cu") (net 3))
 (segment (start 113.344606 102.45607) (end 112.284592 101.396056) (width 0.2) (layer "F.Cu") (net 3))
 (segment (start 144.187304 103.528033) (end 136.494939 103.528033) (width 0.2) (layer "F.Cu") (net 3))
 (segment (start 122.60804 102.342976) (end 113.4577 102.342976) (width 0.2) (layer "F.Cu") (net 3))
 (segment (start 122.60804 102.342976) (end 124.568395 104.303331) (width 0.2) (layer "F.Cu") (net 3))
 (segment (start 107.870772 101.396056) (end 103.690772 101.396056) (width 0.2) (layer "F.Cu") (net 3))
 (segment (start 136.494939 103.528033) (end 131.732999 103.528033) (width 0.2) (layer "F.Cu") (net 3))
 (segment (start 122.60804 107.742976) (end 122.18496 108.166056) (width 0.2) (layer "F.Cu") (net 2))
 (segment (start 122.18496 108.166056) (end 109.811772 108.166056) (width 0.2) (layer "F.Cu") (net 2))
 (segment (start 136.494939 108.128033) (end 133.822403 108.128033) (width 0.2) (layer "F.Cu") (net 2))
 (segment (start 122.60804 107.742976) (end 125.087685 105.263331) (width 0.2) (layer "F.Cu") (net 2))
 (segment (start 133.822403 108.128033) (end 130.957701 105.263331) (width 0.2) (layer "F.Cu") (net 2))
 (segment (start 125.087685 105.263331) (end 130.957701 105.263331) (width 0.2) (layer "F.Cu") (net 2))
 (segment (start 113.367832 107.280921) (end 113.182697 107.466056) (width 0.2) (layer "F.Cu") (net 4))
 (segment (start 113.182697 107.466056) (end 108.785772 107.466056) (width 0.2) (layer "F.Cu") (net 4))
 (segment (start 113.344606 103.47607) (end 112.35462 104.466056) (width 0.2) (layer "F.Cu") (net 1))
 (segment (start 112.35462 104.466056) (end 108.785772 104.466056) (width 0.2) (layer "F.Cu") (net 1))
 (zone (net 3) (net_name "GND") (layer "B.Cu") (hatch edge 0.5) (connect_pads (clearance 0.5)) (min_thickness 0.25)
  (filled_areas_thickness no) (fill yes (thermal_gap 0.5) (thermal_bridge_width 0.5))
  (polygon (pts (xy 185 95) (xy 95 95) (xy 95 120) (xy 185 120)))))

